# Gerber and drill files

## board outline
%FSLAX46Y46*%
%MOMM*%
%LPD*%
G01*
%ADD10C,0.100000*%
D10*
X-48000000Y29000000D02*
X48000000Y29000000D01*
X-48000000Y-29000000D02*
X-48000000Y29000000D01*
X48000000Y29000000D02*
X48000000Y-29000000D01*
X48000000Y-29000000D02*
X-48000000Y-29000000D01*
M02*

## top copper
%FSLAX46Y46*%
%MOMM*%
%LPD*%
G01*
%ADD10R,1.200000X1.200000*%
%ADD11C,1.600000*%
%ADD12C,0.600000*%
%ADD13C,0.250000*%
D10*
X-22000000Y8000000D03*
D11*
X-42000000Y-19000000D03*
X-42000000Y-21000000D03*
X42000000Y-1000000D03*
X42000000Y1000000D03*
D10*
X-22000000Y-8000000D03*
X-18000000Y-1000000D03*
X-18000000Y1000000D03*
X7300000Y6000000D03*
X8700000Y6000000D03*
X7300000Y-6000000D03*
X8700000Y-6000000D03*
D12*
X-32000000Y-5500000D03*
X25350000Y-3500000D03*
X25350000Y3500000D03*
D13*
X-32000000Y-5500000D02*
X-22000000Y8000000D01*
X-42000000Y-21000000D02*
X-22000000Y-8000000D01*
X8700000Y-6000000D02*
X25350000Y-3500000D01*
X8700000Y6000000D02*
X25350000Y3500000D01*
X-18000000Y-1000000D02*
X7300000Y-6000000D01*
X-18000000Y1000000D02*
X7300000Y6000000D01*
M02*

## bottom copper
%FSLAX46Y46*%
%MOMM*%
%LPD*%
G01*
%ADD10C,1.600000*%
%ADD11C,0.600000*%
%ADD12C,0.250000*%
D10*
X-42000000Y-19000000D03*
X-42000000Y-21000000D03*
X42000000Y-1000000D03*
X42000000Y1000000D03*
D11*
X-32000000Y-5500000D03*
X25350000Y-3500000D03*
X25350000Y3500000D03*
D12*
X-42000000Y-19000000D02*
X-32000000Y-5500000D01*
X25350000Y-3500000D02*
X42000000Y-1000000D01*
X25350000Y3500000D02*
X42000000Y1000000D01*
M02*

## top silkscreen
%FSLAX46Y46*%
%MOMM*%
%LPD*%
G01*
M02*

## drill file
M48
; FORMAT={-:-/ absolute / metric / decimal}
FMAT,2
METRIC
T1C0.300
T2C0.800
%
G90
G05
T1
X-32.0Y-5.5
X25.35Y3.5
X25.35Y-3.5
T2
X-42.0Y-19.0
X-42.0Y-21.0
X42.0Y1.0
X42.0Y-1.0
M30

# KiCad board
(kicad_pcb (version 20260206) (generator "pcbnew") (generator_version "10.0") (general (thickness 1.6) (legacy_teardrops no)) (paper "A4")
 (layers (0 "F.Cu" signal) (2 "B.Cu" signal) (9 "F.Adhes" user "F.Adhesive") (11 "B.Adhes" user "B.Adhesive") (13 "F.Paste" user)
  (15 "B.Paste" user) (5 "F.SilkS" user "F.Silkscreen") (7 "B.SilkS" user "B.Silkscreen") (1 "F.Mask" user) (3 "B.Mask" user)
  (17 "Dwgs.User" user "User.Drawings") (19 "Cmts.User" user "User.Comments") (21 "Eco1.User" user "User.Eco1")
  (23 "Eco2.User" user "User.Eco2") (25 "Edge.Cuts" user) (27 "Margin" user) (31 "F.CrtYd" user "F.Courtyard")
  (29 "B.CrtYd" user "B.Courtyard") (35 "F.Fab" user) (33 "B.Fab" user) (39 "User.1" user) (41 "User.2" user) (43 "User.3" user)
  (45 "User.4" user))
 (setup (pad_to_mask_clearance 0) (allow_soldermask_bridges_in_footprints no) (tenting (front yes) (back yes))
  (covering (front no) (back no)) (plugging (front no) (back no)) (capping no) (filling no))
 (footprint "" (layer "F.Cu") (at -22 -8)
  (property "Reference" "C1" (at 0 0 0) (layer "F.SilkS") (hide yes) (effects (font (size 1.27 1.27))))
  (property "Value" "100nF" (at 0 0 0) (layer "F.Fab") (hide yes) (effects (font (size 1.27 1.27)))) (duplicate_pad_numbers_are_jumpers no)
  (pad "1" smd rect (at 0 0) (size 1.2 1.2) (layers "F.Cu" "F.Mask" "F.Paste") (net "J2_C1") (thermal_bridge_angle 45)))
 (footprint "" (layer "F.Cu") (at -42 20)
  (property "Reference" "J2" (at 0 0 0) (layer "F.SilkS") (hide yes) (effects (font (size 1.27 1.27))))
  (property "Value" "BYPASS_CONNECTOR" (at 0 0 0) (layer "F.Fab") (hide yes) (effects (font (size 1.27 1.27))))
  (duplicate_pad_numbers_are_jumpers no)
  (pad "1" thru_hole circle (at 0 -1) (size 1.6 1.6) (drill 0.8) (layers "*.Cu" "*.Mask") (remove_unused_layers no) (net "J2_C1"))
  (pad "2" thru_hole circle (at 0 1) (size 1.6 1.6) (drill 0.8) (layers "*.Cu" "*.Mask") (remove_unused_layers no) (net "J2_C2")))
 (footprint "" (layer "F.Cu") (at 42 0)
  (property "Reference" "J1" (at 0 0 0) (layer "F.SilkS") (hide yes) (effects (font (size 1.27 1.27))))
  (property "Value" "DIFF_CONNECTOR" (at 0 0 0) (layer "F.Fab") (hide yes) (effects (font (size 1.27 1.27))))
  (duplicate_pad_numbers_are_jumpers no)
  (pad "1" thru_hole circle (at 0 1) (size 1.6 1.6) (drill 0.8) (layers "*.Cu" "*.Mask") (remove_unused_layers no) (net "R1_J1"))
  (pad "2" thru_hole circle (at 0 -1) (size 1.6 1.6) (drill 0.8) (layers "*.Cu" "*.Mask") (remove_unused_layers no) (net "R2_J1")))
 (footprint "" (layer "F.Cu") (at -22 8)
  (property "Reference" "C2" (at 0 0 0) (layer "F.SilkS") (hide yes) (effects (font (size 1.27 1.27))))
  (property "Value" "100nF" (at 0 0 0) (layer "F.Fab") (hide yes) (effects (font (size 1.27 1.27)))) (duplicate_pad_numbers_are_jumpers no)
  (pad "1" smd rect (at 0 0) (size 1.2 1.2) (layers "F.Cu" "F.Mask" "F.Paste") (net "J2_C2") (thermal_bridge_angle 45)))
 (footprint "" (layer "F.Cu") (at -18 0)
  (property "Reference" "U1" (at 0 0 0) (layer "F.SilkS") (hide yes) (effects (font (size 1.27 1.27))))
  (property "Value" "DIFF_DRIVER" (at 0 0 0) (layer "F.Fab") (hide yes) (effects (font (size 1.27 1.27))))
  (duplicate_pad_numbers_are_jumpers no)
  (pad "1" smd rect (at 0 1) (size 1.2 1.2) (layers "F.Cu" "F.Mask" "F.Paste") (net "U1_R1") (thermal_bridge_angle 45))
  (pad "2" smd rect (at 0 -1) (size 1.2 1.2) (layers "F.Cu" "F.Mask" "F.Paste") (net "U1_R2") (thermal_bridge_angle 45)))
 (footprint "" (layer "F.Cu") (at 8 -6)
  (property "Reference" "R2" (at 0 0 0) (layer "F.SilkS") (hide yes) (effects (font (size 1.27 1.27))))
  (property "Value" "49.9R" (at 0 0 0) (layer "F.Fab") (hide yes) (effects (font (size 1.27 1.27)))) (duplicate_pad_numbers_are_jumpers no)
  (pad "1" smd rect (at -0.7 0) (size 1.2 1.2) (layers "F.Cu" "F.Mask" "F.Paste") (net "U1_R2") (thermal_bridge_angle 45))
  (pad "2" smd rect (at 0.7 0) (size 1.2 1.2) (layers "F.Cu" "F.Mask" "F.Paste") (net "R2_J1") (thermal_bridge_angle 45)))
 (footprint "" (layer "F.Cu") (at 8 6)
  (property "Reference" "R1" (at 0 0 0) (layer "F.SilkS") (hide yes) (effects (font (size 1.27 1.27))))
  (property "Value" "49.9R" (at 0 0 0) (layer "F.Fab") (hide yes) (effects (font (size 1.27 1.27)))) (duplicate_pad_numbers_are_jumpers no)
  (pad "1" smd rect (at -0.7 0) (size 1.2 1.2) (layers "F.Cu" "F.Mask" "F.Paste") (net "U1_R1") (thermal_bridge_angle 45))
  (pad "2" smd rect (at 0.7 0) (size 1.2 1.2) (layers "F.Cu" "F.Mask" "F.Paste") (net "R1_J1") (thermal_bridge_angle 45)))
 (gr_line (start -48 -29) (end 48 -29) (stroke (width 0.1) (type default)) (layer "Edge.Cuts"))
 (gr_line (start -48 29) (end -48 -29) (stroke (width 0.1) (type default)) (layer "Edge.Cuts"))
 (gr_line (start 48 -29) (end 48 29) (stroke (width 0.1) (type default)) (layer "Edge.Cuts"))
 (gr_line (start 48 29) (end -48 29) (stroke (width 0.1) (type default)) (layer "Edge.Cuts"))
 (segment (start -32 5.5) (end -22 -8) (width 0.25) (layer "F.Cu") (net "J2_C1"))
 (via (at -32 5.5) (size 0.6) (drill 0.3) (layers "F.Cu" "B.Cu") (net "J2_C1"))
 (segment (start -42 19) (end -32 5.5) (width 0.25) (layer "B.Cu") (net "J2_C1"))
 (segment (start -42 21) (end -22 8) (width 0.25) (layer "F.Cu") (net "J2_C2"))
 (segment (start 8.7 6) (end 25.35 3.5) (width 0.25) (layer "F.Cu") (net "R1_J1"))
 (via (at 25.35 3.5) (size 0.6) (drill 0.3) (layers "F.Cu" "B.Cu") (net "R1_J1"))
 (segment (start 25.35 3.5) (end 42 1) (width 0.25) (layer "B.Cu") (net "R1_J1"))
 (segment (start 8.7 -6) (end 25.35 -3.5) (width 0.25) (layer "F.Cu") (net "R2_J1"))
 (via (at 25.35 -3.5) (size 0.6) (drill 0.3) (layers "F.Cu" "B.Cu") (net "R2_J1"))
 (segment (start 25.35 -3.5) (end 42 -1) (width 0.25) (layer "B.Cu") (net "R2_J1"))
 (segment (start -18 1) (end 7.3 6) (width 0.25) (layer "F.Cu") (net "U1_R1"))
 (segment (start -18 -1) (end 7.3 -6) (width 0.25) (layer "F.Cu") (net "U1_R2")))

